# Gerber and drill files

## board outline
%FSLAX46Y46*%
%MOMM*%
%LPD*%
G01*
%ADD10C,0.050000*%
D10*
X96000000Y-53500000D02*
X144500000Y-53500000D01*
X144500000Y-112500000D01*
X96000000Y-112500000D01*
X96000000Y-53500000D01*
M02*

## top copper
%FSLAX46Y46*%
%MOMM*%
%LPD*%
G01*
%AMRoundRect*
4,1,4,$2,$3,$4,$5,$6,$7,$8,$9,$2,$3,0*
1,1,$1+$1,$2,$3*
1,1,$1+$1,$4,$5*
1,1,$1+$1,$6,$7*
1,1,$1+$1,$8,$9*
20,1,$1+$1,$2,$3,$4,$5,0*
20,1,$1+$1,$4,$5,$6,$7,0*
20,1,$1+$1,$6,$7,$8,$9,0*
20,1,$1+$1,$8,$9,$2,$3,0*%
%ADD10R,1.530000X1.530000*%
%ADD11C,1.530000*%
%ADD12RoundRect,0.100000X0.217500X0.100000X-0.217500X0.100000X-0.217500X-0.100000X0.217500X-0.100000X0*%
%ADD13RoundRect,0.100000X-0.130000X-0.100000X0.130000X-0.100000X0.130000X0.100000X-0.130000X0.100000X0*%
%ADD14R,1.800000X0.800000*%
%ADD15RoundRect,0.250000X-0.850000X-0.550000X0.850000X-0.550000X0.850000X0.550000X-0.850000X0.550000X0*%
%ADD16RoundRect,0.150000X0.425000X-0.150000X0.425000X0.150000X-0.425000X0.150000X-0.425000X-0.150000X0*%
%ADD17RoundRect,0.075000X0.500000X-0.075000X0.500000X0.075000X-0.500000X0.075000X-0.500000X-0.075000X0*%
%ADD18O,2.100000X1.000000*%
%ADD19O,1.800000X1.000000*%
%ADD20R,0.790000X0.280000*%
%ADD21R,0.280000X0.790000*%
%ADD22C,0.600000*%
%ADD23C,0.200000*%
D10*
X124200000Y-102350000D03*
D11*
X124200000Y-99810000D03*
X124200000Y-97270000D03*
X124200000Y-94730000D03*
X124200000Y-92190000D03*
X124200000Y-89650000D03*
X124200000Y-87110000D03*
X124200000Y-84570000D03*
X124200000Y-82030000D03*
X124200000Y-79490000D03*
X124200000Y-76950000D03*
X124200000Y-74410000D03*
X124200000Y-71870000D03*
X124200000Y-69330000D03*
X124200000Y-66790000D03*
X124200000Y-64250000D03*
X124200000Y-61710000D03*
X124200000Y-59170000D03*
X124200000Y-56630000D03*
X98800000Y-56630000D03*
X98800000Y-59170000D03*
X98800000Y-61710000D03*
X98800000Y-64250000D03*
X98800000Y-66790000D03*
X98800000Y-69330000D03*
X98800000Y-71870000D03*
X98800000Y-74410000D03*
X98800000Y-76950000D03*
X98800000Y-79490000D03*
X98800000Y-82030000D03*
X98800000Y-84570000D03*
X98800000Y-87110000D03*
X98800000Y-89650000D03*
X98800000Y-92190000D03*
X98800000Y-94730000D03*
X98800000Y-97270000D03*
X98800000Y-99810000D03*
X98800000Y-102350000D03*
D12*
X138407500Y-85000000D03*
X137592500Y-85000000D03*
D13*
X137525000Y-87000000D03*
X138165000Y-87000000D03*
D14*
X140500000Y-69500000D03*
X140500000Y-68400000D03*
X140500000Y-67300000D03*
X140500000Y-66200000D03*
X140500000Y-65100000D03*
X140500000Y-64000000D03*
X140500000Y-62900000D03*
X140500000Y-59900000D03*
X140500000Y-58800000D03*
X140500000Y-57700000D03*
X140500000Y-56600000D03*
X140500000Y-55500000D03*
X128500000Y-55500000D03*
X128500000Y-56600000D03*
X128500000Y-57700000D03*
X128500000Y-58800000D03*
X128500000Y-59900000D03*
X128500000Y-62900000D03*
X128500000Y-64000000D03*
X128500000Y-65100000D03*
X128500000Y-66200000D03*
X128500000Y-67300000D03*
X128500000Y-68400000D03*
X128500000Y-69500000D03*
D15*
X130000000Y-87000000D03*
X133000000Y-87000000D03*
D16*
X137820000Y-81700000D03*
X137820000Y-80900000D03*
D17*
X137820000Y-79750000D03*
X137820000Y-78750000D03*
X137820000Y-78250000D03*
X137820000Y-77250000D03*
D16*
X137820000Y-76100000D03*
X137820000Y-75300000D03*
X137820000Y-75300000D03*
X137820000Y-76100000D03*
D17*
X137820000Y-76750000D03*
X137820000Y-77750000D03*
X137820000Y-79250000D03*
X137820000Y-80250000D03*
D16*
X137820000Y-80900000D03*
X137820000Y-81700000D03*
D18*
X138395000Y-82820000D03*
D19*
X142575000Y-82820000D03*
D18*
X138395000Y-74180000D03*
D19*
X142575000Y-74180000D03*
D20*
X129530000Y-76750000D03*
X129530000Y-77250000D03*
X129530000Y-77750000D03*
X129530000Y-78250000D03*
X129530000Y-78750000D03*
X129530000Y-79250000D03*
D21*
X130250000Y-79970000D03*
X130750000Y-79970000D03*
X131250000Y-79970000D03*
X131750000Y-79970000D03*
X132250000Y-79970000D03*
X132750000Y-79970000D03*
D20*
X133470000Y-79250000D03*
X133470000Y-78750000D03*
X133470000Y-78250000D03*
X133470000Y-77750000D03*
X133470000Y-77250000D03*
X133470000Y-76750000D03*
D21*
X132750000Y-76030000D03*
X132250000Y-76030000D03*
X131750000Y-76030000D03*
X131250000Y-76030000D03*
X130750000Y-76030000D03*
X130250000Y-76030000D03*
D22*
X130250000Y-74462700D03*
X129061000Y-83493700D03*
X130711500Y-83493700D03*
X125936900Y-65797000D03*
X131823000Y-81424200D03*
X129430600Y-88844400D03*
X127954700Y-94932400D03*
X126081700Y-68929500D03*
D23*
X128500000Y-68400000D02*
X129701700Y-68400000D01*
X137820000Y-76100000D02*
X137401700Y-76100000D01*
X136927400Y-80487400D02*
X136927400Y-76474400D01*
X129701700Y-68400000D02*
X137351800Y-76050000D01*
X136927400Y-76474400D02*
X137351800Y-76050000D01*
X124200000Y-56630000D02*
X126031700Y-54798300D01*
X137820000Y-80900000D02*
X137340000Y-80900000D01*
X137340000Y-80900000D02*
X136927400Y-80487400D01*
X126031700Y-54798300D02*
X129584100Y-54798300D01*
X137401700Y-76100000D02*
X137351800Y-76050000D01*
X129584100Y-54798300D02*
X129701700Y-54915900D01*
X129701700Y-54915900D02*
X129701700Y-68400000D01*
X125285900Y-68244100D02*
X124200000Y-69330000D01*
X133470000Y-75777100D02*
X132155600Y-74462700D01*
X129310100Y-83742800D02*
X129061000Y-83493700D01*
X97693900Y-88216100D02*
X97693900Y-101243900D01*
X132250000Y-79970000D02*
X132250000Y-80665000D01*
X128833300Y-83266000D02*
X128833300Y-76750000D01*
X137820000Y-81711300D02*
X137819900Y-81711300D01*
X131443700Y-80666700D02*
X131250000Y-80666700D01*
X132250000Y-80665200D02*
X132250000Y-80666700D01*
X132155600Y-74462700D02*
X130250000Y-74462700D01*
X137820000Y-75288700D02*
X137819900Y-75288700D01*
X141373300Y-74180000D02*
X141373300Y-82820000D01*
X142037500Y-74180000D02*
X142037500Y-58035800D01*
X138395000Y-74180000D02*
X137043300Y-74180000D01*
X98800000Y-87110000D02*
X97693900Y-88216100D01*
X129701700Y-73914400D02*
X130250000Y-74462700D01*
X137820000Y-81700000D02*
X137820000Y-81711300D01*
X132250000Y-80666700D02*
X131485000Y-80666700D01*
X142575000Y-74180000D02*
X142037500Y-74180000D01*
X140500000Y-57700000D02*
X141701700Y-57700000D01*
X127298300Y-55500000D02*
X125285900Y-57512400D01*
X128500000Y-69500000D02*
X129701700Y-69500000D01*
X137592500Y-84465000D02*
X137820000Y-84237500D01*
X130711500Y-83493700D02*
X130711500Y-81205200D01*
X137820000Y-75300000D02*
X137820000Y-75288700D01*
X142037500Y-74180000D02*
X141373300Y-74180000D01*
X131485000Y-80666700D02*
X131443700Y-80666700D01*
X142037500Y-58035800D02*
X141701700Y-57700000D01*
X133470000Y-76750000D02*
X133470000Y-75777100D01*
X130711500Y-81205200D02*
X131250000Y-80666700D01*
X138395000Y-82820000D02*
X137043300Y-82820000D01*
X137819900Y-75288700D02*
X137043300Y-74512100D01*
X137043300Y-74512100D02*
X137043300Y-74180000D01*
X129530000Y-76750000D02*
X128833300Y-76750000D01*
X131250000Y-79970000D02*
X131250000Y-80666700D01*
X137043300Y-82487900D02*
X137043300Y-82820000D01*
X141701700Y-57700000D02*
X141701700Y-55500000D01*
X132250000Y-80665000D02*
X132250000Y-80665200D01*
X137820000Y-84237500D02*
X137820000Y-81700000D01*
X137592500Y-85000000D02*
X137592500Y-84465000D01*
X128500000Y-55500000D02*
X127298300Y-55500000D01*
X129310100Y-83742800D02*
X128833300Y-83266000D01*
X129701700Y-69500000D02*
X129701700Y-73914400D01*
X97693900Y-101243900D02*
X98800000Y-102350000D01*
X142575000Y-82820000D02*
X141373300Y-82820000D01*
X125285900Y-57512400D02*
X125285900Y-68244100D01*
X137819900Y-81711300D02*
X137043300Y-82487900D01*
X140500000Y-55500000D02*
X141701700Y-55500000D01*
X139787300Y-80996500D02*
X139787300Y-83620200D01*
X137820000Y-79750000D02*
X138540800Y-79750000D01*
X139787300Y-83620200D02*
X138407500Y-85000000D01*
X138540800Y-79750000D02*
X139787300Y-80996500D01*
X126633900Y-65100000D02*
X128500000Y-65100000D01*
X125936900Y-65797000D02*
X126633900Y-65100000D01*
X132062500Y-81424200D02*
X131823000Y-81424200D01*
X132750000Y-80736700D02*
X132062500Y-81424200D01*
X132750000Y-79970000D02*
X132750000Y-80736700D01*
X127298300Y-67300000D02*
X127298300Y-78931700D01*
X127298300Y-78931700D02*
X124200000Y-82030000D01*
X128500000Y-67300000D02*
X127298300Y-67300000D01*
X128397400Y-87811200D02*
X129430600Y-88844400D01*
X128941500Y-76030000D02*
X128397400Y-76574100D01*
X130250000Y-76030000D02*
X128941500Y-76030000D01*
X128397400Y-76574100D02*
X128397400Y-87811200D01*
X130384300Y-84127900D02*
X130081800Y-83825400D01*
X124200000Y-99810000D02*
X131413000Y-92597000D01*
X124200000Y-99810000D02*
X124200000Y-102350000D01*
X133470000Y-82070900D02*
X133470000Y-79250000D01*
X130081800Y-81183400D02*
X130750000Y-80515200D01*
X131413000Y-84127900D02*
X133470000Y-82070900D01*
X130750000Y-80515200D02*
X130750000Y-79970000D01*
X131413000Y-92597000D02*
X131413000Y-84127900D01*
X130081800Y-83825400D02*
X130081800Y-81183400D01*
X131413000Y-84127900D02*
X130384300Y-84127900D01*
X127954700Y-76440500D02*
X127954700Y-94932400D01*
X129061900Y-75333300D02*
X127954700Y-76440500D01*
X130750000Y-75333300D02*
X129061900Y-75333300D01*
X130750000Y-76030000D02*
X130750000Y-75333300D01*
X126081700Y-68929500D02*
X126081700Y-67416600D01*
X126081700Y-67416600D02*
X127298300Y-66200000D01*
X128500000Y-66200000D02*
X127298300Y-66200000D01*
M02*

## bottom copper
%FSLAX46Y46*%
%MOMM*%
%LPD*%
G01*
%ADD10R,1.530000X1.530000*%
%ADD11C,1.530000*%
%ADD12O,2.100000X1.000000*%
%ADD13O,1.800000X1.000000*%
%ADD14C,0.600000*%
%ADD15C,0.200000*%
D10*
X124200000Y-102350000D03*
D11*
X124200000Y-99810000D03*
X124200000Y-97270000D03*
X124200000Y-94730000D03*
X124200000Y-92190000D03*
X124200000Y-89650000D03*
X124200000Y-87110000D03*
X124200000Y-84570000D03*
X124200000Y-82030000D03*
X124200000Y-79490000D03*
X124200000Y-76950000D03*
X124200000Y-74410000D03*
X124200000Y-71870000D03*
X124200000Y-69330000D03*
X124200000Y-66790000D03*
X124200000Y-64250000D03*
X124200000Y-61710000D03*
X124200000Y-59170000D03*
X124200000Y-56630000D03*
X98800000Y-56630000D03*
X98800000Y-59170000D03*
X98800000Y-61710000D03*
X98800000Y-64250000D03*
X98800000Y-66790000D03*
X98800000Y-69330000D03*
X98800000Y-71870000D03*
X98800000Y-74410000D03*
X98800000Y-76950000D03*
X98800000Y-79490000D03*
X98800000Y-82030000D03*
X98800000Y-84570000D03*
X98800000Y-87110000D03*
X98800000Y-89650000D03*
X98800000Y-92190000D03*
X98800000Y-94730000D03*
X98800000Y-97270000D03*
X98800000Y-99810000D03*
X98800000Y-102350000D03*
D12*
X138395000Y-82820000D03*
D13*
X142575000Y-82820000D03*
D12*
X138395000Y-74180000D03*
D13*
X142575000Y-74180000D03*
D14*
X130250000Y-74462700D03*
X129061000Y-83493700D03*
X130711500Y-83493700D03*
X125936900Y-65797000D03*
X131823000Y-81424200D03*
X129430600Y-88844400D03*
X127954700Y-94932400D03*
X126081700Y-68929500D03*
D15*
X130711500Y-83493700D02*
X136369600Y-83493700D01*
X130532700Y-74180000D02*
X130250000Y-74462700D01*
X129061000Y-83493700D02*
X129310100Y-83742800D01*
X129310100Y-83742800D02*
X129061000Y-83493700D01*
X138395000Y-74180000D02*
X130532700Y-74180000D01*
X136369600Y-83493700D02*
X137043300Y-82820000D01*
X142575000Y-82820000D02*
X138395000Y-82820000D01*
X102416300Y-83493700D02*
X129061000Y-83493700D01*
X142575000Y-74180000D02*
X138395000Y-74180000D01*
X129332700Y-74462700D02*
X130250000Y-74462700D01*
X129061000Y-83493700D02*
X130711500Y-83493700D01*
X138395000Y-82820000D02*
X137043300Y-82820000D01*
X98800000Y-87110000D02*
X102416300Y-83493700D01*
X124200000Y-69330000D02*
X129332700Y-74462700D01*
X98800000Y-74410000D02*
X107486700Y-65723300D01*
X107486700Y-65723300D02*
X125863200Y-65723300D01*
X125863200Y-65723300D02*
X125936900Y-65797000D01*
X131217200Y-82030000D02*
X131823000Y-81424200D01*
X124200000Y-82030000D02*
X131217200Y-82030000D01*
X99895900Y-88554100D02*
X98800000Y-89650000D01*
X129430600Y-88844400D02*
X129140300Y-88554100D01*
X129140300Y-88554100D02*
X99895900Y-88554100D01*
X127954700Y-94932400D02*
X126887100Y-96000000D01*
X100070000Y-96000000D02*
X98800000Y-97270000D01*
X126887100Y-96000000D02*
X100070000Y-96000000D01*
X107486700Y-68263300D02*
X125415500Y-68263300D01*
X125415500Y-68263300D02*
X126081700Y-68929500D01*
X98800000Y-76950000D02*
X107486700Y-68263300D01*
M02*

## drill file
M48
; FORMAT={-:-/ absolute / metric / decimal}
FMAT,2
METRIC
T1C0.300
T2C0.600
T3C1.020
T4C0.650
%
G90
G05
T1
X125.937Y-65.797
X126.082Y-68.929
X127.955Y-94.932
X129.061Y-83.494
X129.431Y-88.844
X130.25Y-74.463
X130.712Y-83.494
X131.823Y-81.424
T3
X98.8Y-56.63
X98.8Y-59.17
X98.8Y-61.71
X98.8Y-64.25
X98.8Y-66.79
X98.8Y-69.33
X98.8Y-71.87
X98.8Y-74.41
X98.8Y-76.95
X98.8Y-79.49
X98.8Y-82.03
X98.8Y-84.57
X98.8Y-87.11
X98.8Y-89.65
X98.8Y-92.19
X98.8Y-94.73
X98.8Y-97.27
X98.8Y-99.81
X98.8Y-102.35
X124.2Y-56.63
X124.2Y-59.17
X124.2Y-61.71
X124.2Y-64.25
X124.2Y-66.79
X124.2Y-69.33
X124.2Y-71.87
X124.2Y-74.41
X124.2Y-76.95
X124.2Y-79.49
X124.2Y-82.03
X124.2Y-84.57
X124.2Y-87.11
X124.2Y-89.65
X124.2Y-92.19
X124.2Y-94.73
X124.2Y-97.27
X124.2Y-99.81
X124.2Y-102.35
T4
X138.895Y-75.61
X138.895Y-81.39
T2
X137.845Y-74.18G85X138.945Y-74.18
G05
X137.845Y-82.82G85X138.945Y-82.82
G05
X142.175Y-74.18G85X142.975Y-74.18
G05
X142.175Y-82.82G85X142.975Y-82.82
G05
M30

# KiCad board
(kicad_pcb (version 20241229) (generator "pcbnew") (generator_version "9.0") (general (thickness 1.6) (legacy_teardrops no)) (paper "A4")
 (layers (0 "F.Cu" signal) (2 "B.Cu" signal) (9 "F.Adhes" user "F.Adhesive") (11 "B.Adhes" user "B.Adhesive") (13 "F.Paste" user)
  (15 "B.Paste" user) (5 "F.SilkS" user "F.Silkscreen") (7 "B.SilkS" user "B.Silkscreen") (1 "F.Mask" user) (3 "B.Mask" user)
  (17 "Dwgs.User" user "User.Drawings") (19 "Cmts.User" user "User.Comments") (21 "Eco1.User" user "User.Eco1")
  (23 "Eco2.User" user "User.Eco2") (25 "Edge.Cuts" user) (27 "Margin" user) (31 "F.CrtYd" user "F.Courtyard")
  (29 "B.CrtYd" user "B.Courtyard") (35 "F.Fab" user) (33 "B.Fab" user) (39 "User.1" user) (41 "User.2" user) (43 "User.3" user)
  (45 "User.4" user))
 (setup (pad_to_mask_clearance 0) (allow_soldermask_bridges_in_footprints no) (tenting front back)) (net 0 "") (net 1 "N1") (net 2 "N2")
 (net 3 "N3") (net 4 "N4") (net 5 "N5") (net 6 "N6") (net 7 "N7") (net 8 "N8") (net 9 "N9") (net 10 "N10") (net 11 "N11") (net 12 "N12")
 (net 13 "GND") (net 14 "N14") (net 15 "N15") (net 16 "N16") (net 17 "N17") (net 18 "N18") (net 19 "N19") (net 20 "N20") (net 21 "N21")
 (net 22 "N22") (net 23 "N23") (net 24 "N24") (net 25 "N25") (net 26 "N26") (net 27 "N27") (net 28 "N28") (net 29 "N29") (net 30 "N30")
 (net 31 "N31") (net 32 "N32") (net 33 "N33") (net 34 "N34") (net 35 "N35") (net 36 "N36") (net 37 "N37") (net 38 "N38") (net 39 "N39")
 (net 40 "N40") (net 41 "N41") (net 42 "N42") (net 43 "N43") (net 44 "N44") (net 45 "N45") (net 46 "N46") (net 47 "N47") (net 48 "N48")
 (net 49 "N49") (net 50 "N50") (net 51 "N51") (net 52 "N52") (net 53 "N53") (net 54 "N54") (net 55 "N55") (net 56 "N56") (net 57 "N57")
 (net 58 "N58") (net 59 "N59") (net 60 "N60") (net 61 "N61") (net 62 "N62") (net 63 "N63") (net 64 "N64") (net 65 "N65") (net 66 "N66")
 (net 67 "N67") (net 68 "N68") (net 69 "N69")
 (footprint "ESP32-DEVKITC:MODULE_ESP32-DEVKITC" (layer "F.Cu") (at 111.5 79.5 180)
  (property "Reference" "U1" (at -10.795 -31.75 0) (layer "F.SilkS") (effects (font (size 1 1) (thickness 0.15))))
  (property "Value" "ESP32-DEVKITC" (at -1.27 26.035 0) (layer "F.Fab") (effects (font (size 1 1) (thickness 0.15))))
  (pad "1" thru_hole rect (at -12.7 -22.85 180) (size 1.53 1.53) (drill 1.02) (layers "*.Cu" "*.Mask") (remove_unused_layers no)
   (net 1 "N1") (solder_mask_margin 0.102))
  (pad "2" thru_hole circle (at -12.7 -20.31 180) (size 1.53 1.53) (drill 1.02) (layers "*.Cu" "*.Mask") (remove_unused_layers no)
   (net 1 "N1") (solder_mask_margin 0.102))
  (pad "3" thru_hole circle (at -12.7 -17.77 180) (size 1.53 1.53) (drill 1.02) (layers "*.Cu" "*.Mask") (remove_unused_layers no)
   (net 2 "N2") (solder_mask_margin 0.102))
  (pad "4" thru_hole circle (at -12.7 -15.23 180) (size 1.53 1.53) (drill 1.02) (layers "*.Cu" "*.Mask") (remove_unused_layers no)
   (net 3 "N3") (solder_mask_margin 0.102))
  (pad "5" thru_hole circle (at -12.7 -12.69 180) (size 1.53 1.53) (drill 1.02) (layers "*.Cu" "*.Mask") (remove_unused_layers no)
   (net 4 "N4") (solder_mask_margin 0.102))
  (pad "6" thru_hole circle (at -12.7 -10.15 180) (size 1.53 1.53) (drill 1.02) (layers "*.Cu" "*.Mask") (remove_unused_layers no)
   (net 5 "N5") (solder_mask_margin 0.102))
  (pad "7" thru_hole circle (at -12.7 -7.61 180) (size 1.53 1.53) (drill 1.02) (layers "*.Cu" "*.Mask") (remove_unused_layers no)
   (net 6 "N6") (solder_mask_margin 0.102))
  (pad "8" thru_hole circle (at -12.7 -5.07 180) (size 1.53 1.53) (drill 1.02) (layers "*.Cu" "*.Mask") (remove_unused_layers no)
   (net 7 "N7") (solder_mask_margin 0.102))
  (pad "9" thru_hole circle (at -12.7 -2.53 180) (size 1.53 1.53) (drill 1.02) (layers "*.Cu" "*.Mask") (remove_unused_layers no)
   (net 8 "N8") (solder_mask_margin 0.102))
  (pad "10" thru_hole circle (at -12.7 0.01 180) (size 1.53 1.53) (drill 1.02) (layers "*.Cu" "*.Mask") (remove_unused_layers no)
   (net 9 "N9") (solder_mask_margin 0.102))
  (pad "11" thru_hole circle (at -12.7 2.55 180) (size 1.53 1.53) (drill 1.02) (layers "*.Cu" "*.Mask") (remove_unused_layers no)
   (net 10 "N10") (solder_mask_margin 0.102))
  (pad "12" thru_hole circle (at -12.7 5.09 180) (size 1.53 1.53) (drill 1.02) (layers "*.Cu" "*.Mask") (remove_unused_layers no)
   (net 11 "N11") (solder_mask_margin 0.102))
  (pad "13" thru_hole circle (at -12.7 7.63 180) (size 1.53 1.53) (drill 1.02) (layers "*.Cu" "*.Mask") (remove_unused_layers no)
   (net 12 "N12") (solder_mask_margin 0.102))
  (pad "14" thru_hole circle (at -12.7 10.17 180) (size 1.53 1.53) (drill 1.02) (layers "*.Cu" "*.Mask") (remove_unused_layers no)
   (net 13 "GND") (solder_mask_margin 0.102))
  (pad "15" thru_hole circle (at -12.7 12.71 180) (size 1.53 1.53) (drill 1.02) (layers "*.Cu" "*.Mask") (remove_unused_layers no)
   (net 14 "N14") (solder_mask_margin 0.102))
  (pad "16" thru_hole circle (at -12.7 15.25 180) (size 1.53 1.53) (drill 1.02) (layers "*.Cu" "*.Mask") (remove_unused_layers no)
   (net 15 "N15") (solder_mask_margin 0.102))
  (pad "17" thru_hole circle (at -12.7 17.79 180) (size 1.53 1.53) (drill 1.02) (layers "*.Cu" "*.Mask") (remove_unused_layers no)
   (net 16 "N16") (solder_mask_margin 0.102))
  (pad "18" thru_hole circle (at -12.7 20.33 180) (size 1.53 1.53) (drill 1.02) (layers "*.Cu" "*.Mask") (remove_unused_layers no)
   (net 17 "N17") (solder_mask_margin 0.102))
  (pad "19" thru_hole circle (at -12.7 22.87 180) (size 1.53 1.53) (drill 1.02) (layers "*.Cu" "*.Mask") (remove_unused_layers no)
   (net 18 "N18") (solder_mask_margin 0.102))
  (pad "20" thru_hole circle (at 12.7 22.87 180) (size 1.53 1.53) (drill 1.02) (layers "*.Cu" "*.Mask") (remove_unused_layers no)
   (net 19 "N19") (solder_mask_margin 0.102))
  (pad "21" thru_hole circle (at 12.7 20.33 180) (size 1.53 1.53) (drill 1.02) (layers "*.Cu" "*.Mask") (remove_unused_layers no)
   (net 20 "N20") (solder_mask_margin 0.102))
  (pad "22" thru_hole circle (at 12.7 17.79 180) (size 1.53 1.53) (drill 1.02) (layers "*.Cu" "*.Mask") (remove_unused_layers no)
   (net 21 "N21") (solder_mask_margin 0.102))
  (pad "23" thru_hole circle (at 12.7 15.25 180) (size 1.53 1.53) (drill 1.02) (layers "*.Cu" "*.Mask") (remove_unused_layers no)
   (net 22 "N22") (solder_mask_margin 0.102))
  (pad "24" thru_hole circle (at 12.7 12.71 180) (size 1.53 1.53) (drill 1.02) (layers "*.Cu" "*.Mask") (remove_unused_layers no)
   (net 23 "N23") (solder_mask_margin 0.102))
  (pad "25" thru_hole circle (at 12.7 10.17 180) (size 1.53 1.53) (drill 1.02) (layers "*.Cu" "*.Mask") (remove_unused_layers no)
   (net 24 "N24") (solder_mask_margin 0.102))
  (pad "26" thru_hole circle (at 12.7 7.63 180) (size 1.53 1.53) (drill 1.02) (layers "*.Cu" "*.Mask") (remove_unused_layers no)
   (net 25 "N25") (solder_mask_margin 0.102))
  (pad "27" thru_hole circle (at 12.7 5.09 180) (size 1.53 1.53) (drill 1.02) (layers "*.Cu" "*.Mask") (remove_unused_layers no)
   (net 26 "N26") (solder_mask_margin 0.102))
  (pad "28" thru_hole circle (at 12.7 2.55 180) (size 1.53 1.53) (drill 1.02) (layers "*.Cu" "*.Mask") (remove_unused_layers no)
   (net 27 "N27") (solder_mask_margin 0.102))
  (pad "29" thru_hole circle (at 12.7 0.01 180) (size 1.53 1.53) (drill 1.02) (layers "*.Cu" "*.Mask") (remove_unused_layers no)
   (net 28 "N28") (solder_mask_margin 0.102))
  (pad "30" thru_hole circle (at 12.7 -2.53 180) (size 1.53 1.53) (drill 1.02) (layers "*.Cu" "*.Mask") (remove_unused_layers no)
   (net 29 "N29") (solder_mask_margin 0.102))
  (pad "31" thru_hole circle (at 12.7 -5.07 180) (size 1.53 1.53) (drill 1.02) (layers "*.Cu" "*.Mask") (remove_unused_layers no)
   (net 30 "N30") (solder_mask_margin 0.102))
  (pad "32" thru_hole circle (at 12.7 -7.61 180) (size 1.53 1.53) (drill 1.02) (layers "*.Cu" "*.Mask") (remove_unused_layers no)
   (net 13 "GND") (solder_mask_margin 0.102))
  (pad "33" thru_hole circle (at 12.7 -10.15 180) (size 1.53 1.53) (drill 1.02) (layers "*.Cu" "*.Mask") (remove_unused_layers no)
   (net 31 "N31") (solder_mask_margin 0.102))
  (pad "34" thru_hole circle (at 12.7 -12.69 180) (size 1.53 1.53) (drill 1.02) (layers "*.Cu" "*.Mask") (remove_unused_layers no)
   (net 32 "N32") (solder_mask_margin 0.102))
  (pad "35" thru_hole circle (at 12.7 -15.23 180) (size 1.53 1.53) (drill 1.02) (layers "*.Cu" "*.Mask") (remove_unused_layers no)
   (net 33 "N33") (solder_mask_margin 0.102))
  (pad "36" thru_hole circle (at 12.7 -17.77 180) (size 1.53 1.53) (drill 1.02) (layers "*.Cu" "*.Mask") (remove_unused_layers no)
   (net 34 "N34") (solder_mask_margin 0.102))
  (pad "37" thru_hole circle (at 12.7 -20.31 180) (size 1.53 1.53) (drill 1.02) (layers "*.Cu" "*.Mask") (remove_unused_layers no)
   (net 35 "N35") (solder_mask_margin 0.102))
  (pad "38" thru_hole circle (at 12.7 -22.85 180) (size 1.53 1.53) (drill 1.02) (layers "*.Cu" "*.Mask") (remove_unused_layers no)
   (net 13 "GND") (solder_mask_margin 0.102)))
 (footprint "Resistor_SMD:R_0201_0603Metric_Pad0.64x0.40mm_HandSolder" (layer "F.Cu") (at 138 85 180)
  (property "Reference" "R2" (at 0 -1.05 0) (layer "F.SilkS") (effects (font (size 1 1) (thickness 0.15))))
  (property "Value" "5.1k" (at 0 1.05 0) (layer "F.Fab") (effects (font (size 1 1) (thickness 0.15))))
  (pad "" smd roundrect (at -0.4325 0 180) (size 0.458 0.36) (layers "F.Paste") (roundrect_rratio 0.25))
  (pad "" smd roundrect (at 0.4325 0 180) (size 0.458 0.36) (layers "F.Paste") (roundrect_rratio 0.25))
  (pad "1" smd roundrect (at -0.4075 0 180) (size 0.635 0.4) (layers "F.Cu" "F.Mask") (roundrect_rratio 0.25) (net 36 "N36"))
  (pad "2" smd roundrect (at 0.4075 0 180) (size 0.635 0.4) (layers "F.Cu" "F.Mask") (roundrect_rratio 0.25) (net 13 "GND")))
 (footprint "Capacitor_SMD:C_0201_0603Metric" (layer "F.Cu") (at 137.845 87)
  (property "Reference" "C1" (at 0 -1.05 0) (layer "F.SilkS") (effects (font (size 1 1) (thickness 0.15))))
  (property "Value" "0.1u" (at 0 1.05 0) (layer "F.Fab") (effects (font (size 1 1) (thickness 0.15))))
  (pad "" smd roundrect (at -0.345 0) (size 0.318 0.36) (layers "F.Paste") (roundrect_rratio 0.25))
  (pad "" smd roundrect (at 0.345 0) (size 0.318 0.36) (layers "F.Paste") (roundrect_rratio 0.25))
  (pad "1" smd roundrect (at -0.32 0) (size 0.46 0.4) (layers "F.Cu" "F.Mask") (roundrect_rratio 0.25))
  (pad "2" smd roundrect (at 0.32 0) (size 0.46 0.4) (layers "F.Cu" "F.Mask") (roundrect_rratio 0.25)))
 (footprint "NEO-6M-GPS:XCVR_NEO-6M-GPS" (layer "F.Cu") (at 134.5 62.5 180)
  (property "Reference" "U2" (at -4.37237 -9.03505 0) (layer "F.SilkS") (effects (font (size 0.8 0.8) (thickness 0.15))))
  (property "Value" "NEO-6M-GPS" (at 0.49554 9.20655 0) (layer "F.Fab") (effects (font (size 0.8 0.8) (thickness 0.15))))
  (pad "1" smd rect (at -6 -7 180) (size 1.8 0.8) (layers "F.Cu" "F.Mask") (solder_mask_margin 0.102))
  (pad "2" smd rect (at -6 -5.9 180) (size 1.8 0.8) (layers "F.Cu" "F.Mask") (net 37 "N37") (solder_mask_margin 0.102))
  (pad "3" smd rect (at -6 -4.8 180) (size 1.8 0.8) (layers "F.Cu" "F.Mask") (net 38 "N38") (solder_mask_margin 0.102))
  (pad "4" smd rect (at -6 -3.7 180) (size 1.8 0.8) (layers "F.Cu" "F.Mask") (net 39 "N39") (solder_mask_margin 0.102))
  (pad "5" smd rect (at -6 -2.6 180) (size 1.8 0.8) (layers "F.Cu" "F.Mask") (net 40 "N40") (solder_mask_margin 0.102))
  (pad "6" smd rect (at -6 -1.5 180) (size 1.8 0.8) (layers "F.Cu" "F.Mask") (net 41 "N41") (solder_mask_margin 0.102))
  (pad "7" smd rect (at -6 -0.4 180) (size 1.8 0.8) (layers "F.Cu" "F.Mask") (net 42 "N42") (solder_mask_margin 0.102))
  (pad "8" smd rect (at -6 2.6 180) (size 1.8 0.8) (layers "F.Cu" "F.Mask") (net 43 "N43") (solder_mask_margin 0.102))
  (pad "9" smd rect (at -6 3.7 180) (size 1.8 0.8) (layers "F.Cu" "F.Mask") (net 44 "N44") (solder_mask_margin 0.102))
  (pad "10" smd rect (at -6 4.8 180) (size 1.8 0.8) (layers "F.Cu" "F.Mask") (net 13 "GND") (solder_mask_margin 0.102))
  (pad "11" smd rect (at -6 5.9 180) (size 1.8 0.8) (layers "F.Cu" "F.Mask") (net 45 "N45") (solder_mask_margin 0.102))
  (pad "12" smd rect (at -6 7 180) (size 1.8 0.8) (layers "F.Cu" "F.Mask") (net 13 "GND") (solder_mask_margin 0.102))
  (pad "13" smd rect (at 6 7 180) (size 1.8 0.8) (layers "F.Cu" "F.Mask") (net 13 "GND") (solder_mask_margin 0.102))
  (pad "14" smd rect (at 6 5.9 180) (size 1.8 0.8) (layers "F.Cu" "F.Mask") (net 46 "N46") (solder_mask_margin 0.102))
  (pad "15" smd rect (at 6 4.8 180) (size 1.8 0.8) (layers "F.Cu" "F.Mask") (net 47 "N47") (solder_mask_margin 0.102))
  (pad "16" smd rect (at 6 3.7 180) (size 1.8 0.8) (layers "F.Cu" "F.Mask") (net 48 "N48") (solder_mask_margin 0.102))
  (pad "17" smd rect (at 6 2.6 180) (size 1.8 0.8) (layers "F.Cu" "F.Mask") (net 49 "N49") (solder_mask_margin 0.102))
  (pad "18" smd rect (at 6 -0.4 180) (size 1.8 0.8) (layers "F.Cu" "F.Mask") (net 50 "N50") (solder_mask_margin 0.102))
  (pad "19" smd rect (at 6 -1.5 180) (size 1.8 0.8) (layers "F.Cu" "F.Mask") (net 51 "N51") (solder_mask_margin 0.102))
  (pad "20" smd rect (at 6 -2.6 180) (size 1.8 0.8) (layers "F.Cu" "F.Mask") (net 26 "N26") (solder_mask_margin 0.102))
  (pad "21" smd rect (at 6 -3.7 180) (size 1.8 0.8) (layers "F.Cu" "F.Mask") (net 27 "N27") (solder_mask_margin 0.102))
  (pad "22" smd rect (at 6 -4.8 180) (size 1.8 0.8) (layers "F.Cu" "F.Mask") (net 8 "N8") (solder_mask_margin 0.102))
  (pad "23" smd rect (at 6 -5.9 180) (size 1.8 0.8) (layers "F.Cu" "F.Mask") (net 18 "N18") (solder_mask_margin 0.102))
  (pad "24" smd rect (at 6 -7 180) (size 1.8 0.8) (layers "F.Cu" "F.Mask") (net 13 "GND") (solder_mask_margin 0.102)))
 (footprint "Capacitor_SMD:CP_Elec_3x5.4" (layer "F.Cu") (at 131.5 87)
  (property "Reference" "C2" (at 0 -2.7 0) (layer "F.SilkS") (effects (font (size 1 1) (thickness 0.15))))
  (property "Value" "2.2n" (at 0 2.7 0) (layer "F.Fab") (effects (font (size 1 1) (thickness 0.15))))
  (pad "1" smd roundrect (at -1.5 0) (size 2.2 1.6) (layers "F.Cu" "F.Mask" "F.Paste") (roundrect_rratio 0.15625))
  (pad "2" smd roundrect (at 1.5 0) (size 2.2 1.6) (layers "F.Cu" "F.Mask" "F.Paste") (roundrect_rratio 0.15625)))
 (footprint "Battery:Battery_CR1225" (layer "F.Cu") (at 136 103.5)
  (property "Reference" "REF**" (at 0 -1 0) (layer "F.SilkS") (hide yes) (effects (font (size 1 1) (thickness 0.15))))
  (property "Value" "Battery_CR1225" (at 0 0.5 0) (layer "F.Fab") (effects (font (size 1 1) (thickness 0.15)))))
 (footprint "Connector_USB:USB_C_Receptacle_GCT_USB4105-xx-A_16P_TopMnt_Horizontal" (layer "F.Cu") (at 141.5 78.5 90)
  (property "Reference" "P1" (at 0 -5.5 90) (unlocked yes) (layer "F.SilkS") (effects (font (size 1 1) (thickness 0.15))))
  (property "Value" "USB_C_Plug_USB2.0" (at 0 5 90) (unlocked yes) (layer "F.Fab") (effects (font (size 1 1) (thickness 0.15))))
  (pad "" np_thru_hole circle (at -2.89 -2.605 90) (size 0.65 0.65) (drill 0.65) (layers "*.Cu" "*.Mask"))
  (pad "" np_thru_hole circle (at 2.89 -2.605 90) (size 0.65 0.65) (drill 0.65) (layers "*.Cu" "*.Mask"))
  (pad "A1" smd roundrect (at -3.2 -3.68 90) (size 0.6 1.15) (layers "F.Cu" "F.Mask" "F.Paste") (roundrect_rratio 0.25) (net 13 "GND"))
  (pad "A4" smd roundrect (at -2.4 -3.68 90) (size 0.6 1.15) (layers "F.Cu" "F.Mask" "F.Paste") (roundrect_rratio 0.25) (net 18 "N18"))
  (pad "A5" smd roundrect (at -1.25 -3.68 90) (size 0.3 1.15) (layers "F.Cu" "F.Mask" "F.Paste") (roundrect_rratio 0.25) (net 36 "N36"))
  (pad "A6" smd roundrect (at -0.25 -3.68 90) (size 0.3 1.15) (layers "F.Cu" "F.Mask" "F.Paste") (roundrect_rratio 0.25) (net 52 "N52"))
  (pad "A7" smd roundrect (at 0.25 -3.68 90) (size 0.3 1.15) (layers "F.Cu" "F.Mask" "F.Paste") (roundrect_rratio 0.25) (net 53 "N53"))
  (pad "A8" smd roundrect (at 1.25 -3.68 90) (size 0.3 1.15) (layers "F.Cu" "F.Mask" "F.Paste") (roundrect_rratio 0.25))
  (pad "A9" smd roundrect (at 2.4 -3.68 90) (size 0.6 1.15) (layers "F.Cu" "F.Mask" "F.Paste") (roundrect_rratio 0.25) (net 18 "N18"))
  (pad "A12" smd roundrect (at 3.2 -3.68 90) (size 0.6 1.15) (layers "F.Cu" "F.Mask" "F.Paste") (roundrect_rratio 0.25) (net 13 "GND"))
  (pad "B1" smd roundrect (at 3.2 -3.68 90) (size 0.6 1.15) (layers "F.Cu" "F.Mask" "F.Paste") (roundrect_rratio 0.25) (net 13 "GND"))
  (pad "B4" smd roundrect (at 2.4 -3.68 90) (size 0.6 1.15) (layers "F.Cu" "F.Mask" "F.Paste") (roundrect_rratio 0.25) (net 18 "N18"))
  (pad "B5" smd roundrect (at 1.75 -3.68 90) (size 0.3 1.15) (layers "F.Cu" "F.Mask" "F.Paste") (roundrect_rratio 0.25) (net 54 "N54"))
  (pad "B6" smd roundrect (at 0.75 -3.68 90) (size 0.3 1.15) (layers "F.Cu" "F.Mask" "F.Paste") (roundrect_rratio 0.25))
  (pad "B7" smd roundrect (at -0.75 -3.68 90) (size 0.3 1.15) (layers "F.Cu" "F.Mask" "F.Paste") (roundrect_rratio 0.25))
  (pad "B8" smd roundrect (at -1.75 -3.68 90) (size 0.3 1.15) (layers "F.Cu" "F.Mask" "F.Paste") (roundrect_rratio 0.25))
  (pad "B9" smd roundrect (at -2.4 -3.68 90) (size 0.6 1.15) (layers "F.Cu" "F.Mask" "F.Paste") (roundrect_rratio 0.25) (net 18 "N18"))
  (pad "B12" smd roundrect (at -3.2 -3.68 90) (size 0.6 1.15) (layers "F.Cu" "F.Mask" "F.Paste") (roundrect_rratio 0.25) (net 13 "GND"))
  (pad "S1" thru_hole oval (at -4.32 -3.105 90) (size 1 2.1) (drill oval 0.6 1.7) (layers "*.Cu" "*.Mask" "F.Paste")
   (remove_unused_layers no) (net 13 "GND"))
  (pad "S1" thru_hole oval (at -4.32 1.075 90) (size 1 1.8) (drill oval 0.6 1.4) (layers "*.Cu" "*.Mask" "F.Paste")
   (remove_unused_layers no) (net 13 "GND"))
  (pad "S1" thru_hole oval (at 4.32 -3.105 90) (size 1 2.1) (drill oval 0.6 1.7) (layers "*.Cu" "*.Mask" "F.Paste")
   (remove_unused_layers no) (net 13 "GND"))
  (pad "S1" thru_hole oval (at 4.32 1.075 90) (size 1 1.8) (drill oval 0.6 1.4) (layers "*.Cu" "*.Mask" "F.Paste") (remove_unused_layers no)
   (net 13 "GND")))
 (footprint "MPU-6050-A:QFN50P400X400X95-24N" (layer "F.Cu") (at 131.5 78)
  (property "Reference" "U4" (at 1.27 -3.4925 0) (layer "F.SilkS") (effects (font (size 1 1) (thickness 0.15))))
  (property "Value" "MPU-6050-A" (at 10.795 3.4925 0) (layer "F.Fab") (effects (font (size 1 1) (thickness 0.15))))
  (pad "1" smd rect (at -1.97 -1.25) (size 0.79 0.28) (layers "F.Cu" "F.Mask" "F.Paste") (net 13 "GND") (solder_mask_margin 0.102))
  (pad "2" smd rect (at -1.97 -0.75) (size 0.79 0.28) (layers "F.Cu" "F.Mask" "F.Paste") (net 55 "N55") (solder_mask_margin 0.102))
  (pad "3" smd rect (at -1.97 -0.25) (size 0.79 0.28) (layers "F.Cu" "F.Mask" "F.Paste") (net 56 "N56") (solder_mask_margin 0.102))
  (pad "4" smd rect (at -1.97 0.25) (size 0.79 0.28) (layers "F.Cu" "F.Mask" "F.Paste") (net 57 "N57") (solder_mask_margin 0.102))
  (pad "5" smd rect (at -1.97 0.75) (size 0.79 0.28) (layers "F.Cu" "F.Mask" "F.Paste") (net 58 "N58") (solder_mask_margin 0.102))
  (pad "6" smd rect (at -1.97 1.25) (size 0.79 0.28) (layers "F.Cu" "F.Mask" "F.Paste") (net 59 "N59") (solder_mask_margin 0.102))
  (pad "7" smd rect (at -1.25 1.97) (size 0.28 0.79) (layers "F.Cu" "F.Mask" "F.Paste") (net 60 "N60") (solder_mask_margin 0.102))
  (pad "8" smd rect (at -0.75 1.97) (size 0.28 0.79) (layers "F.Cu" "F.Mask" "F.Paste") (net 1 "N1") (solder_mask_margin 0.102))
  (pad "9" smd rect (at -0.25 1.97) (size 0.28 0.79) (layers "F.Cu" "F.Mask" "F.Paste") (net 13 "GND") (solder_mask_margin 0.102))
  (pad "10" smd rect (at 0.25 1.97) (size 0.28 0.79) (layers "F.Cu" "F.Mask" "F.Paste") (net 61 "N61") (solder_mask_margin 0.102))
  (pad "11" smd rect (at 0.75 1.97) (size 0.28 0.79) (layers "F.Cu" "F.Mask" "F.Paste") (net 13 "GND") (solder_mask_margin 0.102))
  (pad "12" smd rect (at 1.25 1.97) (size 0.28 0.79) (layers "F.Cu" "F.Mask" "F.Paste") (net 8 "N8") (solder_mask_margin 0.102))
  (pad "13" smd rect (at 1.97 1.25) (size 0.79 0.28) (layers "F.Cu" "F.Mask" "F.Paste") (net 1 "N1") (solder_mask_margin 0.102))
  (pad "14" smd rect (at 1.97 0.75) (size 0.79 0.28) (layers "F.Cu" "F.Mask" "F.Paste") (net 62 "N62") (solder_mask_margin 0.102))
  (pad "15" smd rect (at 1.97 0.25) (size 0.79 0.28) (layers "F.Cu" "F.Mask" "F.Paste") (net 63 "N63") (solder_mask_margin 0.102))
  (pad "16" smd rect (at 1.97 -0.25) (size 0.79 0.28) (layers "F.Cu" "F.Mask" "F.Paste") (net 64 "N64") (solder_mask_margin 0.102))
  (pad "17" smd rect (at 1.97 -0.75) (size 0.79 0.28) (layers "F.Cu" "F.Mask" "F.Paste") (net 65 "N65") (solder_mask_margin 0.102))
  (pad "18" smd rect (at 1.97 -1.25) (size 0.79 0.28) (layers "F.Cu" "F.Mask" "F.Paste") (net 13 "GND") (solder_mask_margin 0.102))
  (pad "19" smd rect (at 1.25 -1.97) (size 0.28 0.79) (layers "F.Cu" "F.Mask" "F.Paste") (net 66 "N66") (solder_mask_margin 0.102))
  (pad "20" smd rect (at 0.75 -1.97) (size 0.28 0.79) (layers "F.Cu" "F.Mask" "F.Paste") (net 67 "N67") (solder_mask_margin 0.102))
  (pad "21" smd rect (at 0.25 -1.97) (size 0.28 0.79) (layers "F.Cu" "F.Mask" "F.Paste") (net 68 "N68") (solder_mask_margin 0.102))
  (pad "22" smd rect (at -0.25 -1.97) (size 0.28 0.79) (layers "F.Cu" "F.Mask" "F.Paste") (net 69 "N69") (solder_mask_margin 0.102))
  (pad "23" smd rect (at -0.75 -1.97) (size 0.28 0.79) (layers "F.Cu" "F.Mask" "F.Paste") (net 34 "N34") (solder_mask_margin 0.102))
  (pad "24" smd rect (at -1.25 -1.97) (size 0.28 0.79) (layers "F.Cu" "F.Mask" "F.Paste") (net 31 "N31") (solder_mask_margin 0.102))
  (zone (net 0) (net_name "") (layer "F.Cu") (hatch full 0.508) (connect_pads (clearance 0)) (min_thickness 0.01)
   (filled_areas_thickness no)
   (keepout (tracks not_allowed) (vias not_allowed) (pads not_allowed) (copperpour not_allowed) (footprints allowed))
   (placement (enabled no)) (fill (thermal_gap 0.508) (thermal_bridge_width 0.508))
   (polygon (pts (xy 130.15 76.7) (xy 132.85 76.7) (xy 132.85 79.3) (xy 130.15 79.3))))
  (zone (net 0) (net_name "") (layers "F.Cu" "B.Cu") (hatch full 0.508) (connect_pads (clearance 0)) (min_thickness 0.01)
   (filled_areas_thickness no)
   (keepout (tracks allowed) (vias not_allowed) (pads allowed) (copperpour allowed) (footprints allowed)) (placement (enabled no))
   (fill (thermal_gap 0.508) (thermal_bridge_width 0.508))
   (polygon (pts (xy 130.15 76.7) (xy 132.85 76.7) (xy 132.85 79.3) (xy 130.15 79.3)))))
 (gr_rect (start 96 53.5) (end 144.5 112.5) (stroke (width 0.05) (type default)) (fill no) (layer "Edge.Cuts"))
 (segment (start 128.5 68.4) (end 129.7017 68.4) (width 0.2) (layer "F.Cu") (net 18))
 (segment (start 137.82 76.1) (end 137.4017 76.1) (width 0.2) (layer "F.Cu") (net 18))
 (segment (start 136.9274 80.4874) (end 136.9274 76.4744) (width 0.2) (layer "F.Cu") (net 18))
 (segment (start 129.7017 68.4) (end 137.3518 76.05) (width 0.2) (layer "F.Cu") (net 18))
 (segment (start 136.9274 76.4744) (end 137.3518 76.05) (width 0.2) (layer "F.Cu") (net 18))
 (segment (start 124.2 56.63) (end 126.0317 54.7983) (width 0.2) (layer "F.Cu") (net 18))
 (segment (start 137.82 80.9) (end 137.34 80.9) (width 0.2) (layer "F.Cu") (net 18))
 (segment (start 137.34 80.9) (end 136.9274 80.4874) (width 0.2) (layer "F.Cu") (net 18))
 (segment (start 126.0317 54.7983) (end 129.5841 54.7983) (width 0.2) (layer "F.Cu") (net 18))
 (segment (start 137.4017 76.1) (end 137.3518 76.05) (width 0.2) (layer "F.Cu") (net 18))
 (segment (start 129.5841 54.7983) (end 129.7017 54.9159) (width 0.2) (layer "F.Cu") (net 18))
 (segment (start 129.7017 54.9159) (end 129.7017 68.4) (width 0.2) (layer "F.Cu") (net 18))
 (segment (start 125.2859 68.2441) (end 124.2 69.33) (width 0.2) (layer "F.Cu") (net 13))
 (segment (start 133.47 75.7771) (end 132.1556 74.4627) (width 0.2) (layer "F.Cu") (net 13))
 (segment (start 129.3101 83.7428) (end 129.061 83.4937) (width 0.2) (layer "F.Cu") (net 13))
 (segment (start 97.6939 88.2161) (end 97.6939 101.2439) (width 0.2) (layer "F.Cu") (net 13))
 (segment (start 132.25 79.97) (end 132.25 80.665) (width 0.2) (layer "F.Cu") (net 13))
 (segment (start 128.8333 83.266) (end 128.8333 76.75) (width 0.2) (layer "F.Cu") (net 13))
 (segment (start 137.82 81.7113) (end 137.8199 81.7113) (width 0.2) (layer "F.Cu") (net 13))
 (segment (start 131.4437 80.6667) (end 131.25 80.6667) (width 0.2) (layer "F.Cu") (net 13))
 (segment (start 132.25 80.6652) (end 132.25 80.6667) (width 0.2) (layer "F.Cu") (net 13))
 (segment (start 132.1556 74.4627) (end 130.25 74.4627) (width 0.2) (layer "F.Cu") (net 13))
 (segment (start 137.82 75.2887) (end 137.8199 75.2887) (width 0.2) (layer "F.Cu") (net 13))
 (segment (start 141.3733 74.18) (end 141.3733 82.82) (width 0.2) (layer "F.Cu") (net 13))
 (segment (start 142.0375 74.18) (end 142.0375 58.0358) (width 0.2) (layer "F.Cu") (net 13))
 (segment (start 138.395 74.18) (end 137.0433 74.18) (width 0.2) (layer "F.Cu") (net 13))
 (segment (start 98.8 87.11) (end 97.6939 88.2161) (width 0.2) (layer "F.Cu") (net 13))
 (segment (start 129.7017 73.9144) (end 130.25 74.4627) (width 0.2) (layer "F.Cu") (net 13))
 (segment (start 137.82 81.7) (end 137.82 81.7113) (width 0.2) (layer "F.Cu") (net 13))
 (segment (start 132.25 80.6667) (end 131.485 80.6667) (width 0.2) (layer "F.Cu") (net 13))
 (segment (start 142.575 74.18) (end 142.0375 74.18) (width 0.2) (layer "F.Cu") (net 13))
 (segment (start 140.5 57.7) (end 141.7017 57.7) (width 0.2) (layer "F.Cu") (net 13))
 (segment (start 127.2983 55.5) (end 125.2859 57.5124) (width 0.2) (layer "F.Cu") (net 13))
 (segment (start 128.5 69.5) (end 129.7017 69.5) (width 0.2) (layer "F.Cu") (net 13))
 (segment (start 137.5925 84.465) (end 137.82 84.2375) (width 0.2) (layer "F.Cu") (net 13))
 (segment (start 130.7115 83.4937) (end 130.7115 81.2052) (width 0.2) (layer "F.Cu") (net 13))
 (segment (start 137.82 75.3) (end 137.82 75.2887) (width 0.2) (layer "F.Cu") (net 13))
 (segment (start 142.0375 74.18) (end 141.3733 74.18) (width 0.2) (layer "F.Cu") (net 13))
 (segment (start 131.485 80.6667) (end 131.4437 80.6667) (width 0.2) (layer "F.Cu") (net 13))
 (segment (start 142.0375 58.0358) (end 141.7017 57.7) (width 0.2) (layer "F.Cu") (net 13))
 (segment (start 133.47 76.75) (end 133.47 75.7771) (width 0.2) (layer "F.Cu") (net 13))
 (segment (start 130.7115 81.2052) (end 131.25 80.6667) (width 0.2) (layer "F.Cu") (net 13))
 (segment (start 138.395 82.82) (end 137.0433 82.82) (width 0.2) (layer "F.Cu") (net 13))
 (segment (start 137.8199 75.2887) (end 137.0433 74.5121) (width 0.2) (layer "F.Cu") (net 13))
 (segment (start 137.0433 74.5121) (end 137.0433 74.18) (width 0.2) (layer "F.Cu") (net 13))
 (segment (start 129.53 76.75) (end 128.8333 76.75) (width 0.2) (layer "F.Cu") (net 13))
 (segment (start 131.25 79.97) (end 131.25 80.6667) (width 0.2) (layer "F.Cu") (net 13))
 (segment (start 137.0433 82.4879) (end 137.0433 82.82) (width 0.2) (layer "F.Cu") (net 13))
 (segment (start 141.7017 57.7) (end 141.7017 55.5) (width 0.2) (layer "F.Cu") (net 13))
 (segment (start 132.25 80.665) (end 132.25 80.6652) (width 0.2) (layer "F.Cu") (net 13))
 (segment (start 137.82 84.2375) (end 137.82 81.7) (width 0.2) (layer "F.Cu") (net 13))
 (segment (start 137.5925 85) (end 137.5925 84.465) (width 0.2) (layer "F.Cu") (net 13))
 (segment (start 128.5 55.5) (end 127.2983 55.5) (width 0.2) (layer "F.Cu") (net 13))
 (segment (start 129.3101 83.7428) (end 128.8333 83.266) (width 0.2) (layer "F.Cu") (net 13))
 (segment (start 129.7017 69.5) (end 129.7017 73.9144) (width 0.2) (layer "F.Cu") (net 13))
 (segment (start 97.6939 101.2439) (end 98.8 102.35) (width 0.2) (layer "F.Cu") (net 13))
 (segment (start 142.575 82.82) (end 141.3733 82.82) (width 0.2) (layer "F.Cu") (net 13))
 (segment (start 125.2859 57.5124) (end 125.2859 68.2441) (width 0.2) (layer "F.Cu") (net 13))
 (segment (start 137.8199 81.7113) (end 137.0433 82.4879) (width 0.2) (layer "F.Cu") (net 13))
 (segment (start 140.5 55.5) (end 141.7017 55.5) (width 0.2) (layer "F.Cu") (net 13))
 (via (at 130.25 74.4627) (size 0.6) (drill 0.3) (layers "F.Cu" "B.Cu") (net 13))
 (via (at 129.061 83.4937) (size 0.6) (drill 0.3) (layers "F.Cu" "B.Cu") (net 13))
 (via (at 130.7115 83.4937) (size 0.6) (drill 0.3) (layers "F.Cu" "B.Cu") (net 13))
 (segment (start 130.7115 83.4937) (end 136.3696 83.4937) (width 0.2) (layer "B.Cu") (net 13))
 (segment (start 130.5327 74.18) (end 130.25 74.4627) (width 0.2) (layer "B.Cu") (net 13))
 (segment (start 129.061 83.4937) (end 129.3101 83.7428) (width 0.2) (layer "B.Cu") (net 13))
 (segment (start 129.3101 83.7428) (end 129.061 83.4937) (width 0.2) (layer "B.Cu") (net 13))
 (segment (start 138.395 74.18) (end 130.5327 74.18) (width 0.2) (layer "B.Cu") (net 13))
 (segment (start 136.3696 83.4937) (end 137.0433 82.82) (width 0.2) (layer "B.Cu") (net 13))
 (segment (start 142.575 82.82) (end 138.395 82.82) (width 0.2) (layer "B.Cu") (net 13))
 (segment (start 102.4163 83.4937) (end 129.061 83.4937) (width 0.2) (layer "B.Cu") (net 13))
 (segment (start 142.575 74.18) (end 138.395 74.18) (width 0.2) (layer "B.Cu") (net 13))
 (segment (start 129.3327 74.4627) (end 130.25 74.4627) (width 0.2) (layer "B.Cu") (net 13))
 (segment (start 129.061 83.4937) (end 130.7115 83.4937) (width 0.2) (layer "B.Cu") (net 13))
 (segment (start 138.395 82.82) (end 137.0433 82.82) (width 0.2) (layer "B.Cu") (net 13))
 (segment (start 98.8 87.11) (end 102.4163 83.4937) (width 0.2) (layer "B.Cu") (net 13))
 (segment (start 124.2 69.33) (end 129.3327 74.4627) (width 0.2) (layer "B.Cu") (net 13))
 (segment (start 139.7873 80.9965) (end 139.7873 83.6202) (width 0.2) (layer "F.Cu") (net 36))
 (segment (start 137.82 79.75) (end 138.5408 79.75) (width 0.2) (layer "F.Cu") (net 36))
 (segment (start 139.7873 83.6202) (end 138.4075 85) (width 0.2) (layer "F.Cu") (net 36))
 (segment (start 138.5408 79.75) (end 139.7873 80.9965) (width 0.2) (layer "F.Cu") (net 36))
 (segment (start 126.6339 65.1) (end 128.5 65.1) (width 0.2) (layer "F.Cu") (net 26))
 (segment (start 125.9369 65.797) (end 126.6339 65.1) (width 0.2) (layer "F.Cu") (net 26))
 (via (at 125.9369 65.797) (size 0.6) (drill 0.3) (layers "F.Cu" "B.Cu") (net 26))
 (segment (start 98.8 74.41) (end 107.4867 65.7233) (width 0.2) (layer "B.Cu") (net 26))
 (segment (start 107.4867 65.7233) (end 125.8632 65.7233) (width 0.2) (layer "B.Cu") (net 26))
 (segment (start 125.8632 65.7233) (end 125.9369 65.797) (width 0.2) (layer "B.Cu") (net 26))
 (segment (start 132.0625 81.4242) (end 131.823 81.4242) (width 0.2) (layer "F.Cu") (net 8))
 (segment (start 132.75 80.7367) (end 132.0625 81.4242) (width 0.2) (layer "F.Cu") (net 8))
 (segment (start 132.75 79.97) (end 132.75 80.7367) (width 0.2) (layer "F.Cu") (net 8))
 (segment (start 127.2983 67.3) (end 127.2983 78.9317) (width 0.2) (layer "F.Cu") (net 8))
 (segment (start 127.2983 78.9317) (end 124.2 82.03) (width 0.2) (layer "F.Cu") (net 8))
 (segment (start 128.5 67.3) (end 127.2983 67.3) (width 0.2) (layer "F.Cu") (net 8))
 (via (at 131.823 81.4242) (size 0.6) (drill 0.3) (layers "F.Cu" "B.Cu") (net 8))
 (segment (start 131.2172 82.03) (end 131.823 81.4242) (width 0.2) (layer "B.Cu") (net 8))
 (segment (start 124.2 82.03) (end 131.2172 82.03) (width 0.2) (layer "B.Cu") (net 8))
 (segment (start 128.3974 87.8112) (end 129.4306 88.8444) (width 0.2) (layer "F.Cu") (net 31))
 (segment (start 128.9415 76.03) (end 128.3974 76.5741) (width 0.2) (layer "F.Cu") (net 31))
 (segment (start 130.25 76.03) (end 128.9415 76.03) (width 0.2) (layer "F.Cu") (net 31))
 (segment (start 128.3974 76.5741) (end 128.3974 87.8112) (width 0.2) (layer "F.Cu") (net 31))
 (via (at 129.4306 88.8444) (size 0.6) (drill 0.3) (layers "F.Cu" "B.Cu") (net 31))
 (segment (start 99.8959 88.5541) (end 98.8 89.65) (width 0.2) (layer "B.Cu") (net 31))
 (segment (start 129.4306 88.8444) (end 129.1403 88.5541) (width 0.2) (layer "B.Cu") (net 31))
 (segment (start 129.1403 88.5541) (end 99.8959 88.5541) (width 0.2) (layer "B.Cu") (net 31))
 (segment (start 130.3843 84.1279) (end 130.0818 83.8254) (width 0.2) (layer "F.Cu") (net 1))
 (segment (start 124.2 99.81) (end 131.413 92.597) (width 0.2) (layer "F.Cu") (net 1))
 (segment (start 124.2 99.81) (end 124.2 102.35) (width 0.2) (layer "F.Cu") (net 1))
 (segment (start 133.47 82.0709) (end 133.47 79.25) (width 0.2) (layer "F.Cu") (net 1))
 (segment (start 130.0818 81.1834) (end 130.75 80.5152) (width 0.2) (layer "F.Cu") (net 1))
 (segment (start 131.413 84.1279) (end 133.47 82.0709) (width 0.2) (layer "F.Cu") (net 1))
 (segment (start 130.75 80.5152) (end 130.75 79.97) (width 0.2) (layer "F.Cu") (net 1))
 (segment (start 131.413 92.597) (end 131.413 84.1279) (width 0.2) (layer "F.Cu") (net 1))
 (segment (start 130.0818 83.8254) (end 130.0818 81.1834) (width 0.2) (layer "F.Cu") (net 1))
 (segment (start 131.413 84.1279) (end 130.3843 84.1279) (width 0.2) (layer "F.Cu") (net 1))
 (segment (start 127.9547 76.4405) (end 127.9547 94.9324) (width 0.2) (layer "F.Cu") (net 34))
 (segment (start 129.0619 75.3333) (end 127.9547 76.4405) (width 0.2) (layer "F.Cu") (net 34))
 (segment (start 130.75 75.3333) (end 129.0619 75.3333) (width 0.2) (layer "F.Cu") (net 34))
 (segment (start 130.75 76.03) (end 130.75 75.3333) (width 0.2) (layer "F.Cu") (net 34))
 (via (at 127.9547 94.9324) (size 0.6) (drill 0.3) (layers "F.Cu" "B.Cu") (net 34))
 (segment (start 127.9547 94.9324) (end 126.8871 96) (width 0.2) (layer "B.Cu") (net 34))
 (segment (start 100.07 96) (end 98.8 97.27) (width 0.2) (layer "B.Cu") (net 34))
 (segment (start 126.8871 96) (end 100.07 96) (width 0.2) (layer "B.Cu") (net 34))
 (segment (start 126.0817 68.9295) (end 126.0817 67.4166) (width 0.2) (layer "F.Cu") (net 27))
 (segment (start 126.0817 67.4166) (end 127.2983 66.2) (width 0.2) (layer "F.Cu") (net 27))
 (segment (start 128.5 66.2) (end 127.2983 66.2) (width 0.2) (layer "F.Cu") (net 27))
 (via (at 126.0817 68.9295) (size 0.6) (drill 0.3) (layers "F.Cu" "B.Cu") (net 27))
 (segment (start 107.4867 68.2633) (end 125.4155 68.2633) (width 0.2) (layer "B.Cu") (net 27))
 (segment (start 125.4155 68.2633) (end 126.0817 68.9295) (width 0.2) (layer "B.Cu") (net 27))
 (segment (start 98.8 76.95) (end 107.4867 68.2633) (width 0.2) (layer "B.Cu") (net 27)))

